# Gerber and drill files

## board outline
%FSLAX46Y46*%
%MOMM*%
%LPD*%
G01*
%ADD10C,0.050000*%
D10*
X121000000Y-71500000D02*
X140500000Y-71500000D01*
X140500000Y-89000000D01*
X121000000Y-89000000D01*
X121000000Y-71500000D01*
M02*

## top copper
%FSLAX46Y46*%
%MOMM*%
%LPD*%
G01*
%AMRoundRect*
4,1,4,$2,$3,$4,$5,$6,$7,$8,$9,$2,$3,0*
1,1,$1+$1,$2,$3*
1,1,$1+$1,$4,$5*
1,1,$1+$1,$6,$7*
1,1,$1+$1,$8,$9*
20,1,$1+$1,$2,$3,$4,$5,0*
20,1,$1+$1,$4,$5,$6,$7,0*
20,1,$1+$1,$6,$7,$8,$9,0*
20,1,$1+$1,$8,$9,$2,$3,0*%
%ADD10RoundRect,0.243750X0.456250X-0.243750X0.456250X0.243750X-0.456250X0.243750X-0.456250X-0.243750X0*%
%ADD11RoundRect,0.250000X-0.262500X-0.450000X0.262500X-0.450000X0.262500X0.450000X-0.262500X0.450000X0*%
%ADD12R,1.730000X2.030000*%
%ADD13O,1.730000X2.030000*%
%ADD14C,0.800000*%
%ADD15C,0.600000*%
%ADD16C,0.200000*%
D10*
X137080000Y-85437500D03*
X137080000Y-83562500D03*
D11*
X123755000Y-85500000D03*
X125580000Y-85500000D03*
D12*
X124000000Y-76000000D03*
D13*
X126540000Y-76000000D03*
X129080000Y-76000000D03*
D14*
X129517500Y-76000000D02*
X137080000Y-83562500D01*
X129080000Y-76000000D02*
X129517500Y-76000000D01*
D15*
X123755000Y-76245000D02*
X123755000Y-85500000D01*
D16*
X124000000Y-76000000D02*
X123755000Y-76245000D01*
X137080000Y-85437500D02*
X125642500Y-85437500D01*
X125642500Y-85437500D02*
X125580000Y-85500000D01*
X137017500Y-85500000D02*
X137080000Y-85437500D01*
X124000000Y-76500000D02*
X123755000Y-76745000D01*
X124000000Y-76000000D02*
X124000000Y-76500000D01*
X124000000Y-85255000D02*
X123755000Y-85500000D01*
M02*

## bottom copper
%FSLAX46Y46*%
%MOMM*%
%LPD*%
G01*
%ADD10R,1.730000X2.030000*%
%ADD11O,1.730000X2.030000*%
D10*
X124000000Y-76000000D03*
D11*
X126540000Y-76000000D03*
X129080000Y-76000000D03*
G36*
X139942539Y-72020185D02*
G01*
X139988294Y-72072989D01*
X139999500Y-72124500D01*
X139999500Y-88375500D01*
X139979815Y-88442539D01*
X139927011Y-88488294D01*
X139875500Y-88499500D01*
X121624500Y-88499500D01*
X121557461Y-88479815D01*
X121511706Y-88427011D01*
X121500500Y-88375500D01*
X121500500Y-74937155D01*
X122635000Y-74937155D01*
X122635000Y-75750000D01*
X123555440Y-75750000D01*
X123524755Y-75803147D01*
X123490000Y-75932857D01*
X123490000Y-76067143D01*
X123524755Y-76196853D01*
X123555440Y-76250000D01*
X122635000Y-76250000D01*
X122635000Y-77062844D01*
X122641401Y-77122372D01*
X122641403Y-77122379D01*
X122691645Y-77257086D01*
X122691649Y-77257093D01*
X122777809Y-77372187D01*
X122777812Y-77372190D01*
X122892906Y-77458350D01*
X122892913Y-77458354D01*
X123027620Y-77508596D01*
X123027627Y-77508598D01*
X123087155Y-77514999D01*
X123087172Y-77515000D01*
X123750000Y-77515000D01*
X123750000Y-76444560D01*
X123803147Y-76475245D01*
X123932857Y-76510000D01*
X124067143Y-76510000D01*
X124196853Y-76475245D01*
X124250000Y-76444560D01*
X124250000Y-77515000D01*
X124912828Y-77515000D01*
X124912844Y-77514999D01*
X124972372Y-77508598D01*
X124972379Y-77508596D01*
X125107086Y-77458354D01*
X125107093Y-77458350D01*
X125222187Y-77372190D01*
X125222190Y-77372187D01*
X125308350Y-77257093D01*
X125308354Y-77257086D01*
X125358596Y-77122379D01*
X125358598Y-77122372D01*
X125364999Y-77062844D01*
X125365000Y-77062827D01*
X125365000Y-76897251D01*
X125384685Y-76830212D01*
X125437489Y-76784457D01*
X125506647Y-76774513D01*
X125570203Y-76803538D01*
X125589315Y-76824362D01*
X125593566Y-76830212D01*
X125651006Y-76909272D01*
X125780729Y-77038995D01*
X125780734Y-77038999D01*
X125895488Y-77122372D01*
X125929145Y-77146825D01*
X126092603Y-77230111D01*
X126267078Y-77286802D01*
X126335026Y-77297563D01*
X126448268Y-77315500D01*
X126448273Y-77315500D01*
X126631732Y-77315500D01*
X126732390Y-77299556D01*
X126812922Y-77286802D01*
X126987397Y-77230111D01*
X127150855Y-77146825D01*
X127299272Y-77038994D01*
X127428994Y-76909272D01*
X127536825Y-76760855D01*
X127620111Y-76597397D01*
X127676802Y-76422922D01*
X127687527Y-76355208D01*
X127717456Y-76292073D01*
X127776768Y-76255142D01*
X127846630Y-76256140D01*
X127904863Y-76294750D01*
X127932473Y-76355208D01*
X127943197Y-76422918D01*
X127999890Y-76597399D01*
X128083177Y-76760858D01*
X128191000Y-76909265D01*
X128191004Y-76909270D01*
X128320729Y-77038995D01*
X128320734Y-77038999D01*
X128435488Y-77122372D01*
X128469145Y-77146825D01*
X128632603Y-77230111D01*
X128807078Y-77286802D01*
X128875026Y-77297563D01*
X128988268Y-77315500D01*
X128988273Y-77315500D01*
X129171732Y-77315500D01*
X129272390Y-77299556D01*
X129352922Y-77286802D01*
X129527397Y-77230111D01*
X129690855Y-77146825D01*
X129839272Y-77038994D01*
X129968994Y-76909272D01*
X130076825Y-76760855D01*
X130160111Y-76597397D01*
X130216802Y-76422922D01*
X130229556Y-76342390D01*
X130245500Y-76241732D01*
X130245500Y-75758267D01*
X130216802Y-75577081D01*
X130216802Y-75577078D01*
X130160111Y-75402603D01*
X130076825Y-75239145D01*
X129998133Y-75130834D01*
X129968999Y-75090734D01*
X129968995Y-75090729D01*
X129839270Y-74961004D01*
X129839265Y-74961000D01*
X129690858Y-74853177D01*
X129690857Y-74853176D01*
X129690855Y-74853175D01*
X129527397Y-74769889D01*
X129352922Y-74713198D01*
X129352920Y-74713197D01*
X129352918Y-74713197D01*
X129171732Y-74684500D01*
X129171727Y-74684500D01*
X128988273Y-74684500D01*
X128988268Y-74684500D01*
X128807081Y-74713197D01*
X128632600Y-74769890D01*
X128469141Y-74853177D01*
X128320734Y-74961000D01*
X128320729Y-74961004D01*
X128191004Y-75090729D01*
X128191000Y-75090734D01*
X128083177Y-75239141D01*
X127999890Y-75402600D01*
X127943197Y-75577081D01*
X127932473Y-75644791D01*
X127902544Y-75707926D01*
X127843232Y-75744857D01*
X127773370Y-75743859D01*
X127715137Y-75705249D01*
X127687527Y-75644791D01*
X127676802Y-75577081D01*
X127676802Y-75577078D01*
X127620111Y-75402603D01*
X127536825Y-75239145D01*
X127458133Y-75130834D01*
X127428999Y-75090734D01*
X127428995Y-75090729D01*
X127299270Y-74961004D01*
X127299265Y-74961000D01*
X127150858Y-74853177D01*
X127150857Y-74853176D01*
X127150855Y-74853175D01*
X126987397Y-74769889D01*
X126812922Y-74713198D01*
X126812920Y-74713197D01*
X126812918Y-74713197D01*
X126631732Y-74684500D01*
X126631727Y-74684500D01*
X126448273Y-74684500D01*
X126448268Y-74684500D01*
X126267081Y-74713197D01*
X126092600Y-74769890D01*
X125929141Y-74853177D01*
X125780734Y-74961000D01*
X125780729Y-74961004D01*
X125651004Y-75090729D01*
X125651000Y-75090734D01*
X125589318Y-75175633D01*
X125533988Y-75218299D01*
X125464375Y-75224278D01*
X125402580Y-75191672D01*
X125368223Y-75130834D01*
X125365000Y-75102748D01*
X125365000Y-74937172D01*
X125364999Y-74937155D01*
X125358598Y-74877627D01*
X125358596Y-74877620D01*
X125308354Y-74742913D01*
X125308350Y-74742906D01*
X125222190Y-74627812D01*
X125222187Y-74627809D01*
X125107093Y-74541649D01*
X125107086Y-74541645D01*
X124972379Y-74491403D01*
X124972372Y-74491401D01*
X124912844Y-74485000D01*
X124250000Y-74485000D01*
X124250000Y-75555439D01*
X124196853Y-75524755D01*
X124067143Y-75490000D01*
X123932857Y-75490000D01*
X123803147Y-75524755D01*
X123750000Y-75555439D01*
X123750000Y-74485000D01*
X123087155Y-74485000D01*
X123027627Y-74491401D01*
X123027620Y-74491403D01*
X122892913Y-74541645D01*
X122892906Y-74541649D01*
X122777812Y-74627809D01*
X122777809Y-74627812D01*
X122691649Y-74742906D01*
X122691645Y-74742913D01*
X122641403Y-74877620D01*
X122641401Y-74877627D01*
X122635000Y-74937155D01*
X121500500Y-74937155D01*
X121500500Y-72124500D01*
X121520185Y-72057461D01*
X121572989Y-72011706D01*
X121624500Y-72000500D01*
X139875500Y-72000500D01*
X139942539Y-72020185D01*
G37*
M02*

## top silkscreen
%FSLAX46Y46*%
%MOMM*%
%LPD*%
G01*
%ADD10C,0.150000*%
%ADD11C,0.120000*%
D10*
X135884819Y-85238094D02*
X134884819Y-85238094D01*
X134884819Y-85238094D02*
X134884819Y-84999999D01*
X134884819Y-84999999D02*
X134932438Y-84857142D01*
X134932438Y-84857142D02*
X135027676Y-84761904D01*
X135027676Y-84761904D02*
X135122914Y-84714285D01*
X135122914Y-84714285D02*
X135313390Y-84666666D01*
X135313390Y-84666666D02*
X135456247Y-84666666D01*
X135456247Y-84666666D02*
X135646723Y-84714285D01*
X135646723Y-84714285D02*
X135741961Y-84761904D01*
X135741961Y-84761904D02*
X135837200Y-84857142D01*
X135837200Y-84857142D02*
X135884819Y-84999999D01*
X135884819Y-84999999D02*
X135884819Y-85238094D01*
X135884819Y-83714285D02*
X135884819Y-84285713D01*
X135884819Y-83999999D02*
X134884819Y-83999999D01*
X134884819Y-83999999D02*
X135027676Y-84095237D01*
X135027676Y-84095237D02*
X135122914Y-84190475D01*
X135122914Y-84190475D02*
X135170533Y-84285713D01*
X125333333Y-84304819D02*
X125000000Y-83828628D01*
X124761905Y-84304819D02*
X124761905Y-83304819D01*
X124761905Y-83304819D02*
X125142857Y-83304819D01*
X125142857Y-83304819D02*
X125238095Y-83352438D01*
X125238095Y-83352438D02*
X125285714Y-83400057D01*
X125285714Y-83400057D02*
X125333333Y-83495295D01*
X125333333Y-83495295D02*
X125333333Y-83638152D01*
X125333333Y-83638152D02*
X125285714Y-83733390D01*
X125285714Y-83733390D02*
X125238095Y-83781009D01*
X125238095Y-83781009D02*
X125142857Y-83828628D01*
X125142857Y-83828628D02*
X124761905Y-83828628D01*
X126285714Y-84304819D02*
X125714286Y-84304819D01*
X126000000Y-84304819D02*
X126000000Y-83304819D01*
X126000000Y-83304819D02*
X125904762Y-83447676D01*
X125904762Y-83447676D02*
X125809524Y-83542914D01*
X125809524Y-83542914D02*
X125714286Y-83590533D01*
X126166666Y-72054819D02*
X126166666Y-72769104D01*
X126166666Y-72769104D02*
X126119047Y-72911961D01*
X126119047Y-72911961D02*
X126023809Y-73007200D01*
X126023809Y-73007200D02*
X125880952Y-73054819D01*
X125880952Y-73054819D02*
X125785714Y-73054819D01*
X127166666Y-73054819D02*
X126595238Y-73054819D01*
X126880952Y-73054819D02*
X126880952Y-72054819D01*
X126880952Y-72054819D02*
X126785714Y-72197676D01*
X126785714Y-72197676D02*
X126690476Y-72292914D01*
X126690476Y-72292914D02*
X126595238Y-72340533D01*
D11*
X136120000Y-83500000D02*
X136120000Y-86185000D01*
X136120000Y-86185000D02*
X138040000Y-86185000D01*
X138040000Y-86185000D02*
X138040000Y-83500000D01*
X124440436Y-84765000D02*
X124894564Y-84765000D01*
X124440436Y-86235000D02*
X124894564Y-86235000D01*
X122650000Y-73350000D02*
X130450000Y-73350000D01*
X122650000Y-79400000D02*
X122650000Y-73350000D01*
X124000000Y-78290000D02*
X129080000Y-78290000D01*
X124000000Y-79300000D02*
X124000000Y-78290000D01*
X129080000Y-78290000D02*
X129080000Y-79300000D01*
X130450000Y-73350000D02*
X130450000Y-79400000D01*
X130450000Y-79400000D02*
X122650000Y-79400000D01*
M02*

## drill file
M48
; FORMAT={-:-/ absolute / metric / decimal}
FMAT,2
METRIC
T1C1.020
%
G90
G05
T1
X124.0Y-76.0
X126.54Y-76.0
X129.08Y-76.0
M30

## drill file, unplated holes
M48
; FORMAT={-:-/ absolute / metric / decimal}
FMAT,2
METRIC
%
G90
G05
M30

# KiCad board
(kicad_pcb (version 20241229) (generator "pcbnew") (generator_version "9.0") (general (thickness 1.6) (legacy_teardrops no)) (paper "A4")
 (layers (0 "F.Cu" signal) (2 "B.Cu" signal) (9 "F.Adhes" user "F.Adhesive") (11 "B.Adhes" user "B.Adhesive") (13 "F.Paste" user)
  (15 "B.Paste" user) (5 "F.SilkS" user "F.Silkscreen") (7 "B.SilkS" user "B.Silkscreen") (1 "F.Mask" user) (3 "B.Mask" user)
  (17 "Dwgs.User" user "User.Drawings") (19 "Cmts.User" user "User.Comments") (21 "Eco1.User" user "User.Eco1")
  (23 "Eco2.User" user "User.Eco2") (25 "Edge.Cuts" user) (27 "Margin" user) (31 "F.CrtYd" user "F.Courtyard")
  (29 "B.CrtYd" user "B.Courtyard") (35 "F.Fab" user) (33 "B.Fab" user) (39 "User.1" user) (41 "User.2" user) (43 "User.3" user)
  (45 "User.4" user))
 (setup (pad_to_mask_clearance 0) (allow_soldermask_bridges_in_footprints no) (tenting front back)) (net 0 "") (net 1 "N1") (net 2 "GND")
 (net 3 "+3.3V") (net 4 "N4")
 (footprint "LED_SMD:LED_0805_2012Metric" (layer "F.Cu") (at 137.08 84.5 90)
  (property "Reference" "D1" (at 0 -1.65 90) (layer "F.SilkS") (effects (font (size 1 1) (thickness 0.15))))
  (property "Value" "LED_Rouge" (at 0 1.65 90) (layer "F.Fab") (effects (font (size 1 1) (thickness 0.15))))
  (fp_line (start 1 -0.96) (end -1.685 -0.96) (stroke (width 0.12) (type solid)) (layer "F.SilkS"))
  (fp_line (start -1.685 -0.96) (end -1.685 0.96) (stroke (width 0.12) (type solid)) (layer "F.SilkS"))
  (fp_line (start -1.685 0.96) (end 1 0.96) (stroke (width 0.12) (type solid)) (layer "F.SilkS"))
  (pad "1" smd roundrect (at -0.9375 0 90) (size 0.975 1.4) (layers "F.Cu" "F.Mask" "F.Paste") (roundrect_rratio 0.25) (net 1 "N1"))
  (pad "2" smd roundrect (at 0.9375 0 90) (size 0.975 1.4) (layers "F.Cu" "F.Mask" "F.Paste") (roundrect_rratio 0.25) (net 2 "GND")))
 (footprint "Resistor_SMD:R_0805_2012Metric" (layer "F.Cu") (at 124.6675 85.5)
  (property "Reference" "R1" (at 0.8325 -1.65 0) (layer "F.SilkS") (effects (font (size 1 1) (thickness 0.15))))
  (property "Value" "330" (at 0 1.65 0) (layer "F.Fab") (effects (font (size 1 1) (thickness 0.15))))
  (fp_line (start -0.227064 -0.735) (end 0.227064 -0.735) (stroke (width 0.12) (type solid)) (layer "F.SilkS"))
  (fp_line (start -0.227064 0.735) (end 0.227064 0.735) (stroke (width 0.12) (type solid)) (layer "F.SilkS"))
  (pad "1" smd roundrect (at -0.9125 0) (size 1.025 1.4) (layers "F.Cu" "F.Mask" "F.Paste") (roundrect_rratio 0.243902) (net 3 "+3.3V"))
  (pad "2" smd roundrect (at 0.9125 0) (size 1.025 1.4) (layers "F.Cu" "F.Mask" "F.Paste") (roundrect_rratio 0.243902) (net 1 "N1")))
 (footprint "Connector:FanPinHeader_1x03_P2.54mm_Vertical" (layer "F.Cu") (at 124 76)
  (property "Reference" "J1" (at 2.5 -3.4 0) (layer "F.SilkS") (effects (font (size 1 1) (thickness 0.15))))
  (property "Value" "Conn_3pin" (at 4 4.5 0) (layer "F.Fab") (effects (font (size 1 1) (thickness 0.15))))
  (fp_line (start -1.35 -2.65) (end 6.45 -2.65) (stroke (width 0.12) (type solid)) (layer "F.SilkS"))
  (fp_line (start -1.35 3.4) (end -1.35 -2.65) (stroke (width 0.12) (type solid)) (layer "F.SilkS"))
  (fp_line (start 0 2.29) (end 5.08 2.29) (stroke (width 0.12) (type solid)) (layer "F.SilkS"))
  (fp_line (start 0 3.3) (end 0 2.29) (stroke (width 0.12) (type solid)) (layer "F.SilkS"))
  (fp_line (start 5.08 2.29) (end 5.08 3.3) (stroke (width 0.12) (type solid)) (layer "F.SilkS"))
  (fp_line (start 6.45 -2.65) (end 6.45 3.4) (stroke (width 0.12) (type solid)) (layer "F.SilkS"))
  (fp_line (start 6.45 3.4) (end -1.35 3.4) (stroke (width 0.12) (type solid)) (layer "F.SilkS"))
  (pad "1" thru_hole rect (at 0 0 90) (size 2.03 1.73) (drill 1.02) (layers "*.Cu" "*.Mask") (remove_unused_layers no) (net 3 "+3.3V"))
  (pad "2" thru_hole oval (at 2.54 0 90) (size 2.03 1.73) (drill 1.02) (layers "*.Cu" "*.Mask") (remove_unused_layers no) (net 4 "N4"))
  (pad "3" thru_hole oval (at 5.08 0 90) (size 2.03 1.73) (drill 1.02) (layers "*.Cu" "*.Mask") (remove_unused_layers no) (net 2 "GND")))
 (gr_rect (start 121 71.5) (end 140.5 89) (stroke (width 0.05) (type default)) (fill no) (layer "Edge.Cuts"))
 (segment (start 137.08 85.4375) (end 125.6425 85.4375) (width 0.2) (layer "F.Cu") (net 1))
 (segment (start 125.6425 85.4375) (end 125.58 85.5) (width 0.2) (layer "F.Cu") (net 1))
 (segment (start 137.0175 85.5) (end 137.08 85.4375) (width 0.2) (layer "F.Cu") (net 1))
 (segment (start 129.08 76) (end 129.5175 76) (width 0.8) (layer "F.Cu") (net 2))
 (segment (start 129.5175 76) (end 137.08 83.5625) (width 0.8) (layer "F.Cu") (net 2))
 (segment (start 124 76.5) (end 123.755 76.745) (width 0.2) (layer "F.Cu") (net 3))
 (segment (start 124 76) (end 123.755 76.245) (width 0.2) (layer "F.Cu") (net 3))
 (segment (start 124 76) (end 124 76.5) (width 0.2) (layer "F.Cu") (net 3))
 (segment (start 124 85.255) (end 123.755 85.5) (width 0.2) (layer "F.Cu") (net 3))
 (segment (start 123.755 76.245) (end 123.755 85.5) (width 0.6) (layer "F.Cu") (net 3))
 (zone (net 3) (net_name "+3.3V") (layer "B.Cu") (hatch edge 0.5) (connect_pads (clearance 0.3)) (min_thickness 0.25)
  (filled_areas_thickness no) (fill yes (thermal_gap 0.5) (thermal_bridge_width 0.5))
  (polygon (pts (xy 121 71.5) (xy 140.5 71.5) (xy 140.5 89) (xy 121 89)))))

